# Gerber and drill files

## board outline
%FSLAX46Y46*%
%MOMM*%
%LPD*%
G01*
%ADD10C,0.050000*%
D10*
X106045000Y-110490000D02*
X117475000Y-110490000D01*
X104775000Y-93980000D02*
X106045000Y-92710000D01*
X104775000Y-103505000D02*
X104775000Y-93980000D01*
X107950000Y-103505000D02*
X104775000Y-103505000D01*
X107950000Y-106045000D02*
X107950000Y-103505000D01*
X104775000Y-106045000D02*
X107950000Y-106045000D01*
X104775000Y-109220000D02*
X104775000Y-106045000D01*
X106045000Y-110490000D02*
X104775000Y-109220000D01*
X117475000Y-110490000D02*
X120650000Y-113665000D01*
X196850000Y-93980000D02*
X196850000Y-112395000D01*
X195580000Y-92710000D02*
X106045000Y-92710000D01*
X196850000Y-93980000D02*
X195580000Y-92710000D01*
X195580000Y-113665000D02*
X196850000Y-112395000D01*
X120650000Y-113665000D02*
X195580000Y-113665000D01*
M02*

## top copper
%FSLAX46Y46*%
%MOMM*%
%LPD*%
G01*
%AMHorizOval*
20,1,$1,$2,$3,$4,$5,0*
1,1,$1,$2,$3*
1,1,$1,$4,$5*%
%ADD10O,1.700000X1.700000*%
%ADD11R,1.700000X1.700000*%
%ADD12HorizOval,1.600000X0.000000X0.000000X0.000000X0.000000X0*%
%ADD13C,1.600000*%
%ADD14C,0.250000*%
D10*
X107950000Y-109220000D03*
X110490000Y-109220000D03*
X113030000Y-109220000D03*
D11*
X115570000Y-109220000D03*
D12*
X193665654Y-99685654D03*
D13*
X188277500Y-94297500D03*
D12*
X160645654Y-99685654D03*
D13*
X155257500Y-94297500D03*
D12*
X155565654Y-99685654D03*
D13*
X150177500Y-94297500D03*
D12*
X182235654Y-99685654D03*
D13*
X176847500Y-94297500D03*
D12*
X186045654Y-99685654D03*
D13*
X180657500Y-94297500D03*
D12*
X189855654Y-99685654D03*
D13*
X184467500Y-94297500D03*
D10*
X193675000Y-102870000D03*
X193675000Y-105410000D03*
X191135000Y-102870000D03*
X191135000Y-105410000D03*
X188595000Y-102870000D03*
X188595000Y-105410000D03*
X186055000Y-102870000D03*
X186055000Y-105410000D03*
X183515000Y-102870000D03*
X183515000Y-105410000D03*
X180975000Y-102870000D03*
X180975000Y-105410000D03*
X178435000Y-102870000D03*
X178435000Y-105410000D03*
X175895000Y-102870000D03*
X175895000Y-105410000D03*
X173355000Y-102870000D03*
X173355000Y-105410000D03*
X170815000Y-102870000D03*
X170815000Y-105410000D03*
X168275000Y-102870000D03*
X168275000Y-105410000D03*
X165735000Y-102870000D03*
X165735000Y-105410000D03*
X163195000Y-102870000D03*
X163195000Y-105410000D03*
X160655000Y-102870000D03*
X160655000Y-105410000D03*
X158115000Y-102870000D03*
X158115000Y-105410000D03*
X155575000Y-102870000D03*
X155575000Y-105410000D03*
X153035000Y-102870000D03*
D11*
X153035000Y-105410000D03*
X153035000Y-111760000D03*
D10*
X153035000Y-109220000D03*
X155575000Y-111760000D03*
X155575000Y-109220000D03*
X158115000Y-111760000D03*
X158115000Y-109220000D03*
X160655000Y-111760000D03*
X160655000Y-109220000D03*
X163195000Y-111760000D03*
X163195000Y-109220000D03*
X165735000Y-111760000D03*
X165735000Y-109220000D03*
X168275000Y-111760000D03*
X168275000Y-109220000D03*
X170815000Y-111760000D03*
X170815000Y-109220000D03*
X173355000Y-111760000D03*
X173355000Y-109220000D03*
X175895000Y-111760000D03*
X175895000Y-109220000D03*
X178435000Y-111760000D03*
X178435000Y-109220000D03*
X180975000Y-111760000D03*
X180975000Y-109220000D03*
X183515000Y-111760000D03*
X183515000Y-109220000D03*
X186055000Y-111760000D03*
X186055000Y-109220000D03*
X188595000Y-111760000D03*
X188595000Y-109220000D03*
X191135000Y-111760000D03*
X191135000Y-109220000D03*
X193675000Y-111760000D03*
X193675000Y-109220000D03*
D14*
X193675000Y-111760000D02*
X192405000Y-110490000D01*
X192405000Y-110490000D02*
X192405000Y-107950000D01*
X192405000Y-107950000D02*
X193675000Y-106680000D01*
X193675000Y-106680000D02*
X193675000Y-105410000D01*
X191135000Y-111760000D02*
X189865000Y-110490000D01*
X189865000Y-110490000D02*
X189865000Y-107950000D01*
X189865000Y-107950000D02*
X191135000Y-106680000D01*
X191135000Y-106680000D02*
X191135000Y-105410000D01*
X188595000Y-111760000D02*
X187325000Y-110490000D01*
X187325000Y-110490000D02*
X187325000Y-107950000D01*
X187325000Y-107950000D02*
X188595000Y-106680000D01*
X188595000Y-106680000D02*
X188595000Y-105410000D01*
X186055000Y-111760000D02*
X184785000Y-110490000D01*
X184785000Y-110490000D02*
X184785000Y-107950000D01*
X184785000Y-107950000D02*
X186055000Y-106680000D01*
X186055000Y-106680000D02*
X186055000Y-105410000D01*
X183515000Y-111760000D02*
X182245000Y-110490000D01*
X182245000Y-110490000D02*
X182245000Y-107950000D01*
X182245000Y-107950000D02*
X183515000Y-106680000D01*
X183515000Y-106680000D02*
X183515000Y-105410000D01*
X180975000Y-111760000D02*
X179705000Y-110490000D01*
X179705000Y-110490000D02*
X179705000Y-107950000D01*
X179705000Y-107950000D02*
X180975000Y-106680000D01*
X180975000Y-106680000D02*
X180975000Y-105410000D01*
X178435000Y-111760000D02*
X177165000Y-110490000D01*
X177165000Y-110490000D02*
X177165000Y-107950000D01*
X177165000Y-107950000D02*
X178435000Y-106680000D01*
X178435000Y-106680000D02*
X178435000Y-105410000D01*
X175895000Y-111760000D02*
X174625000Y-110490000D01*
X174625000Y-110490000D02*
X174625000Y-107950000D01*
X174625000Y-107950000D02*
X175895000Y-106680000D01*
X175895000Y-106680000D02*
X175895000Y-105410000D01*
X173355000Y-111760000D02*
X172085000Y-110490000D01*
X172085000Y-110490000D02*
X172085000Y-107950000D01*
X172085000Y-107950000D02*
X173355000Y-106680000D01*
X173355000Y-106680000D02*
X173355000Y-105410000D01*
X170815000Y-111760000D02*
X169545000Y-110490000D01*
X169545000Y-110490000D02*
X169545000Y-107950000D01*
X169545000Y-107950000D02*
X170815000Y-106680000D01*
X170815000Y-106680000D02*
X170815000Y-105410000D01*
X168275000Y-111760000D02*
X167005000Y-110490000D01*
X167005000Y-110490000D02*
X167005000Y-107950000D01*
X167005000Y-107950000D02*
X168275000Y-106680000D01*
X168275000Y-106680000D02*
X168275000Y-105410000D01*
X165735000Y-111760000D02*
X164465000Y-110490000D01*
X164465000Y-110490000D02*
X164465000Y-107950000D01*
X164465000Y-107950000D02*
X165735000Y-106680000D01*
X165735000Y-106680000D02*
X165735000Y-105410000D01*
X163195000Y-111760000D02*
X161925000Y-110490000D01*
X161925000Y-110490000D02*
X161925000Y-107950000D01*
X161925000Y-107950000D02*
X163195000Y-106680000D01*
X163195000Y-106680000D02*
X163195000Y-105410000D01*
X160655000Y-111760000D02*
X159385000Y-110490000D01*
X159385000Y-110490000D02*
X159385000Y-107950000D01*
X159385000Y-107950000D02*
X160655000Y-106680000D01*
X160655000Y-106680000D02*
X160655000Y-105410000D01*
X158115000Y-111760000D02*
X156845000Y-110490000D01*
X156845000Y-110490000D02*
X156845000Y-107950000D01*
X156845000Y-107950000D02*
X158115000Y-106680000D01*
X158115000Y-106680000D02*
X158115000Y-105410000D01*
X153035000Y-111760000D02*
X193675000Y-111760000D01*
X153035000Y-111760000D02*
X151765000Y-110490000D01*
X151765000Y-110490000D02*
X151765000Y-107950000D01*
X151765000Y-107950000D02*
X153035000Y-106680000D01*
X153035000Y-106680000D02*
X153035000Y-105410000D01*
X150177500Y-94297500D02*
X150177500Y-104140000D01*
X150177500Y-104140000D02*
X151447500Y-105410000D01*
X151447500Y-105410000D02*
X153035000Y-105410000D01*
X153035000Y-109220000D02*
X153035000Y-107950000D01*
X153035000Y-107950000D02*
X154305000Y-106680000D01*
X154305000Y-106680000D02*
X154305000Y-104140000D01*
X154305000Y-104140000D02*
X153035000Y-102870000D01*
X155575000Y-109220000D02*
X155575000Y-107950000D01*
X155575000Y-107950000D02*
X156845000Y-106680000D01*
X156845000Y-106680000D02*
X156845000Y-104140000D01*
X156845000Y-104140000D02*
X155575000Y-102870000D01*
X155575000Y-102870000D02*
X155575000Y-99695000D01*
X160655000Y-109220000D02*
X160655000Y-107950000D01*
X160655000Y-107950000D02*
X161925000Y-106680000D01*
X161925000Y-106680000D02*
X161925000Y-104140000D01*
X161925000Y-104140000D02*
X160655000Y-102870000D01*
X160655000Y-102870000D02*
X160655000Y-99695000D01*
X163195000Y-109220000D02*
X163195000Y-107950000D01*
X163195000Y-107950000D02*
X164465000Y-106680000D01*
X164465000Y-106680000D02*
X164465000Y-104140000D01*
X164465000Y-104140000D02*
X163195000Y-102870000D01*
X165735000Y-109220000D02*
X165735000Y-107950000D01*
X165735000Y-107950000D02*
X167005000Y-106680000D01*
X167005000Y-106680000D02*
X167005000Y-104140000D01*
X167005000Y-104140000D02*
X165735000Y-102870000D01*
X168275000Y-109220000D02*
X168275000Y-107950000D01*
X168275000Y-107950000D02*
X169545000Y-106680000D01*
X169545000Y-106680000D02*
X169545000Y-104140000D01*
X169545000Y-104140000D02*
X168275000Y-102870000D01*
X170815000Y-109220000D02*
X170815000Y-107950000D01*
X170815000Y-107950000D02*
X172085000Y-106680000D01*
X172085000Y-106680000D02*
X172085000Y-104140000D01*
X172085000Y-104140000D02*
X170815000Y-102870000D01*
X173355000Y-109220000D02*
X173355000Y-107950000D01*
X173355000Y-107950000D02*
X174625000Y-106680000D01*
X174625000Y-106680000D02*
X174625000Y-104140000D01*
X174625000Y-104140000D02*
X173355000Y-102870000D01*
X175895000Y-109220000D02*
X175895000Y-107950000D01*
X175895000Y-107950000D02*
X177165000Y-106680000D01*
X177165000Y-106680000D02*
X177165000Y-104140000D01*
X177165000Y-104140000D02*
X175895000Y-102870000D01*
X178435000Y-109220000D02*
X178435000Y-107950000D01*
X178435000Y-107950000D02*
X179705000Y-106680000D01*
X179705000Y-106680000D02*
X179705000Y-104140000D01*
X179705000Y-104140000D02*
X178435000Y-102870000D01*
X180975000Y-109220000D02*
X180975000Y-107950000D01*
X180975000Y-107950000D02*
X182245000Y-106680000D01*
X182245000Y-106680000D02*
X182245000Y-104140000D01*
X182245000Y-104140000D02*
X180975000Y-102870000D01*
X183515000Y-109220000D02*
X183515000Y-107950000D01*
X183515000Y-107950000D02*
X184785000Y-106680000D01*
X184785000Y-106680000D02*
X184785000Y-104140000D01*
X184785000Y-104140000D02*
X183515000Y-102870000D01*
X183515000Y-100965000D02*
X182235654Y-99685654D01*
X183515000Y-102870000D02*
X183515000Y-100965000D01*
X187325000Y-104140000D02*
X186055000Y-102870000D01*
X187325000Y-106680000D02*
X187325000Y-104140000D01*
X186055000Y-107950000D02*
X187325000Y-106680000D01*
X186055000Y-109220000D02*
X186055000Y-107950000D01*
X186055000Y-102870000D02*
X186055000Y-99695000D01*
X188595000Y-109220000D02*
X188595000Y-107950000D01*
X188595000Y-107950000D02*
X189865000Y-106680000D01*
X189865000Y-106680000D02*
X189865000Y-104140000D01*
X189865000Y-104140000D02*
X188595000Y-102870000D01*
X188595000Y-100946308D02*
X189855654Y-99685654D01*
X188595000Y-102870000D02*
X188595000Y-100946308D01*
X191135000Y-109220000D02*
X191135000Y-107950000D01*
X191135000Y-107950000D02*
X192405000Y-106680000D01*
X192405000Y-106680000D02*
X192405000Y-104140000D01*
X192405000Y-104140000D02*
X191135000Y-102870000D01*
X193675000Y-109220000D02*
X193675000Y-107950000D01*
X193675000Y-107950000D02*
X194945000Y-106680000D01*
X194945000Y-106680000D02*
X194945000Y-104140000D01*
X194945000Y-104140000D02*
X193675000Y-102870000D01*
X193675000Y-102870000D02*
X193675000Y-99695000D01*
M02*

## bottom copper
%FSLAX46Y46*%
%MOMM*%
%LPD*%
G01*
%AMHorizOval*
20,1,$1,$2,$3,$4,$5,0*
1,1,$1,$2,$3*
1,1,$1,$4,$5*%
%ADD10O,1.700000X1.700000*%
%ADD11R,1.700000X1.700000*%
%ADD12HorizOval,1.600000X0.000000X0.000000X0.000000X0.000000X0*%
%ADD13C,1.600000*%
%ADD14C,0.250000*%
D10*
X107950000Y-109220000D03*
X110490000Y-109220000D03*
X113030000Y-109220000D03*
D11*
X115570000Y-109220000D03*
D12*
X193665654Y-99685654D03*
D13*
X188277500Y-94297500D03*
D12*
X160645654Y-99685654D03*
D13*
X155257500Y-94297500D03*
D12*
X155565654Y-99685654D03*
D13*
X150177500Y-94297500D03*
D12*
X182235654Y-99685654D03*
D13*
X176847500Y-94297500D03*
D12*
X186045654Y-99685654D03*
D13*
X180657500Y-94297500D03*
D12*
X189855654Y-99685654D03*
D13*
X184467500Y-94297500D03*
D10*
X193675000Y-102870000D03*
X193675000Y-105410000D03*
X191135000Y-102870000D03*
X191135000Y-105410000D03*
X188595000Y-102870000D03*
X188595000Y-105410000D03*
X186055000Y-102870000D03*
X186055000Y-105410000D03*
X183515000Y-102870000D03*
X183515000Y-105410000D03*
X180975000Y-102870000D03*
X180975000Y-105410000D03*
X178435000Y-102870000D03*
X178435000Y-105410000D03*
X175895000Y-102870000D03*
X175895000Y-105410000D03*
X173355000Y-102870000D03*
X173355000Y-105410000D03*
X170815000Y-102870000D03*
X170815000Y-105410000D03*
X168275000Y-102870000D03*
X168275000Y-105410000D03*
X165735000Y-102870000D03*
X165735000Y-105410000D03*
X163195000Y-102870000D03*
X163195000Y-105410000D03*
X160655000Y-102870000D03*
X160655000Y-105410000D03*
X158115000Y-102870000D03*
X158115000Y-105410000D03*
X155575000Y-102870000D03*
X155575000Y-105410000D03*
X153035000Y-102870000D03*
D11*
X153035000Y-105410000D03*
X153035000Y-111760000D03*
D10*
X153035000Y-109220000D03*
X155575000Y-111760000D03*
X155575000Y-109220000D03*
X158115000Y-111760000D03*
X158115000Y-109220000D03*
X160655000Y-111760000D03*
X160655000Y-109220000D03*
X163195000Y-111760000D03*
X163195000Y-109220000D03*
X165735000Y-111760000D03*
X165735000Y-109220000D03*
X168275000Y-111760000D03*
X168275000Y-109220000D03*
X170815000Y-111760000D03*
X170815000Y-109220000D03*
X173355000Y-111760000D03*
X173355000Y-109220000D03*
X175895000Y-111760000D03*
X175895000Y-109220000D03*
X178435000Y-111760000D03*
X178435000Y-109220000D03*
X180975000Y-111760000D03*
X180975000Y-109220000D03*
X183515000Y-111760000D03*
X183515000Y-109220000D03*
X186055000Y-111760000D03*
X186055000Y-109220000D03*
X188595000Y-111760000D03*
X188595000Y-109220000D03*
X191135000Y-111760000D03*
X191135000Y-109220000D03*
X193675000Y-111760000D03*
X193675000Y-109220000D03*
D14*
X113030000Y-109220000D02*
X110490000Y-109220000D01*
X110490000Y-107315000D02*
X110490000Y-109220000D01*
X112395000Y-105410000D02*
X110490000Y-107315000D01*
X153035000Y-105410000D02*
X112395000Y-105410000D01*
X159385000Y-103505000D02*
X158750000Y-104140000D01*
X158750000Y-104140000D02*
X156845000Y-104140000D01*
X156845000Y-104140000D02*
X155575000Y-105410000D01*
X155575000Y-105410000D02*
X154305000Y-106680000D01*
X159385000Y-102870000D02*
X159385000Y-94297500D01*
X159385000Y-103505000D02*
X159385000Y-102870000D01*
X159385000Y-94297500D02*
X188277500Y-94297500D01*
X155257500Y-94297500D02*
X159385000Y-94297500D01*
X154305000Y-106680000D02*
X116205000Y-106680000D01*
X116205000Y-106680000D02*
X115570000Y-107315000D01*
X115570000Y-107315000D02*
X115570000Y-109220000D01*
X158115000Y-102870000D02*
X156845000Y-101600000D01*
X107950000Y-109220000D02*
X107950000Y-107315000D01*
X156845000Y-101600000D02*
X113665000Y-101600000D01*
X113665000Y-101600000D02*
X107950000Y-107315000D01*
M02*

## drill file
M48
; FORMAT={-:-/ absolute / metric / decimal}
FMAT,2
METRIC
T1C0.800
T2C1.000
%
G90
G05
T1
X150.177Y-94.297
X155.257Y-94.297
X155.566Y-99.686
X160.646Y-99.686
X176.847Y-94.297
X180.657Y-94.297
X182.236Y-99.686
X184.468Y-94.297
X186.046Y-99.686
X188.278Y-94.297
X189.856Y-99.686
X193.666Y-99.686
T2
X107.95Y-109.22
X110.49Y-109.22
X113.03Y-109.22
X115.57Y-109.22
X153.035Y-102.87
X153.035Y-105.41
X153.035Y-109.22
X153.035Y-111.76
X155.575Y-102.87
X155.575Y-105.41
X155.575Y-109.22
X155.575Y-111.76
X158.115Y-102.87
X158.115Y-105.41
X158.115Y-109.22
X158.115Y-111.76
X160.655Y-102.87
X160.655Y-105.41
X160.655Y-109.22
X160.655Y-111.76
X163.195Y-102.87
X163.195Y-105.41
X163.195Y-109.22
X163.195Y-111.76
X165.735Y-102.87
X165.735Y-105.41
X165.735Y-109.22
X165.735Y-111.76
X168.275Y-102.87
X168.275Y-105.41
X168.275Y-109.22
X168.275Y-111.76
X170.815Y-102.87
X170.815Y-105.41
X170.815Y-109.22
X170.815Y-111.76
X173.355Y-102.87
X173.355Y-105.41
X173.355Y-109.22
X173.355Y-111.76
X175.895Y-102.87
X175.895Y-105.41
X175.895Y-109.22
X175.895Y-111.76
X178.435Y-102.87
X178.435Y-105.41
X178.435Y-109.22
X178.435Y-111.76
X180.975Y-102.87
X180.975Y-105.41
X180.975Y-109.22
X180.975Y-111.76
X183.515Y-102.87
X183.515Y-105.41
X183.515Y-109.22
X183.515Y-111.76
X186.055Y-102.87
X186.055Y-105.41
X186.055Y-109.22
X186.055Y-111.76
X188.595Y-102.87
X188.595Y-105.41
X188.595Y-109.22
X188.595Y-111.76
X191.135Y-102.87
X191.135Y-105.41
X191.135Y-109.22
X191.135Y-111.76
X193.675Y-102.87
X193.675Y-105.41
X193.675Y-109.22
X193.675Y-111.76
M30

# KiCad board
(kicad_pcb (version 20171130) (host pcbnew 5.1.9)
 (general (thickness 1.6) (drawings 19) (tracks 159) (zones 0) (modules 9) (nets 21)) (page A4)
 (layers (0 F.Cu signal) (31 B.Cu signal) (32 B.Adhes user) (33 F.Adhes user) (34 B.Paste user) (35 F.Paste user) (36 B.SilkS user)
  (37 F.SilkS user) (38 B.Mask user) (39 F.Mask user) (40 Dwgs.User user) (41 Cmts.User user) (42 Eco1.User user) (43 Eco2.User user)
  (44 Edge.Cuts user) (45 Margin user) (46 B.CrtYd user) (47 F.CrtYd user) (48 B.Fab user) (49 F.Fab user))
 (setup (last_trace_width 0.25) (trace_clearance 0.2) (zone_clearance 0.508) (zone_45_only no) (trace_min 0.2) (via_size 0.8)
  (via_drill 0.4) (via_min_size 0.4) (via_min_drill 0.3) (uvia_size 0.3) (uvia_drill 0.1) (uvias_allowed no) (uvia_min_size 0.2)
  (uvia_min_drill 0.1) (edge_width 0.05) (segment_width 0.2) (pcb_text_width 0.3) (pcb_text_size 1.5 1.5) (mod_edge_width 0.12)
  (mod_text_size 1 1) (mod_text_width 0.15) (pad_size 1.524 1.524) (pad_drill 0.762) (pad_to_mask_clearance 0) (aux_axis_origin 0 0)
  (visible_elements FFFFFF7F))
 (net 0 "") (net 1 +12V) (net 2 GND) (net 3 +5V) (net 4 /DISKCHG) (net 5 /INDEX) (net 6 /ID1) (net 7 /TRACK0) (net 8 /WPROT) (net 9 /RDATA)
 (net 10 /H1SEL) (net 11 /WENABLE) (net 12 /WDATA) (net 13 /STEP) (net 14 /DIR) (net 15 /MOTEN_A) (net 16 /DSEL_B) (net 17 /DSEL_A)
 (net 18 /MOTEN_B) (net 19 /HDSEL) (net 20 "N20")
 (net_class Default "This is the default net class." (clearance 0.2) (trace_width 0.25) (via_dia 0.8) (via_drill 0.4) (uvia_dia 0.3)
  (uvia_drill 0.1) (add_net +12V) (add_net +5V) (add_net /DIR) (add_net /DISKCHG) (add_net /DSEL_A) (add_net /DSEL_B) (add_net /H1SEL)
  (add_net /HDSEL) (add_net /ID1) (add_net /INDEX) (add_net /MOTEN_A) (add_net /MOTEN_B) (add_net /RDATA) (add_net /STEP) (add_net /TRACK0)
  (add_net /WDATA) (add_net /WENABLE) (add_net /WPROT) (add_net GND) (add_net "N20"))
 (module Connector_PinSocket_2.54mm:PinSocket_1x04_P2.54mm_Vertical (layer B.Cu) (at 115.57 109.22 90)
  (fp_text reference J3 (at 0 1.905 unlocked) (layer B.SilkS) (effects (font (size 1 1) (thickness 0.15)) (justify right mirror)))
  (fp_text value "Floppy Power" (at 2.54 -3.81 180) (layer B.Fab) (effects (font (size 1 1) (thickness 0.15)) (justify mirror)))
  (pad 4 thru_hole oval (at 0 -7.62 90) (size 1.7 1.7) (drill 1) (layers *.Cu *.Mask) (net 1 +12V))
  (pad 3 thru_hole oval (at 0 -5.08 90) (size 1.7 1.7) (drill 1) (layers *.Cu *.Mask) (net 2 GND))
  (pad 2 thru_hole oval (at 0 -2.54 90) (size 1.7 1.7) (drill 1) (layers *.Cu *.Mask) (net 2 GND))
  (pad 1 thru_hole rect (at 0 0 90) (size 1.7 1.7) (drill 1) (layers *.Cu *.Mask) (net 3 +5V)))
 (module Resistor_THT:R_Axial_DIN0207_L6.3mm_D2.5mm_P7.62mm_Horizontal (layer F.Cu) (at 188.2775 94.2975 315)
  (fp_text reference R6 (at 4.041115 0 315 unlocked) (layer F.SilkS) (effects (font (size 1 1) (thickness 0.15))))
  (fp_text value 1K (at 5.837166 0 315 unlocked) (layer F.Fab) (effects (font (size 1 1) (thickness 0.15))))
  (pad 2 thru_hole oval (at 7.62 0 315) (size 1.6 1.6) (drill 0.8) (layers *.Cu *.Mask) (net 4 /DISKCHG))
  (pad 1 thru_hole circle (at 0 0 315) (size 1.6 1.6) (drill 0.8) (layers *.Cu *.Mask) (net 3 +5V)))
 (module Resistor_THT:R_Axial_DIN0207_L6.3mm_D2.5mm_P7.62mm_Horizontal (layer F.Cu) (at 155.2575 94.2975 315)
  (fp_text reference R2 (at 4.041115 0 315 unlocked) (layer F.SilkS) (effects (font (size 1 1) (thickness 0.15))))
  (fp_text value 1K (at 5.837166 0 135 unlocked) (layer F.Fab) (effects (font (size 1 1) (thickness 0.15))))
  (pad 2 thru_hole oval (at 7.62 0 315) (size 1.6 1.6) (drill 0.8) (layers *.Cu *.Mask) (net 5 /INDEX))
  (pad 1 thru_hole circle (at 0 0 315) (size 1.6 1.6) (drill 0.8) (layers *.Cu *.Mask) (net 3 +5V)))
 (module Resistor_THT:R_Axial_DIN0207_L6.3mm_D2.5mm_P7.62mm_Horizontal (layer F.Cu) (at 150.1775 94.2975 315)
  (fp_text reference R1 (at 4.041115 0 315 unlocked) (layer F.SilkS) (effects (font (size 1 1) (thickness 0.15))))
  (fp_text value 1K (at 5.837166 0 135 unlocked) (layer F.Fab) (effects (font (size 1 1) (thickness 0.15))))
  (pad 2 thru_hole oval (at 7.62 0 315) (size 1.6 1.6) (drill 0.8) (layers *.Cu *.Mask) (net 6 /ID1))
  (pad 1 thru_hole circle (at 0 0 315) (size 1.6 1.6) (drill 0.8) (layers *.Cu *.Mask) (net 2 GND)))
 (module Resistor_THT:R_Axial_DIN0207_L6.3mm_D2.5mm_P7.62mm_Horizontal (layer F.Cu) (at 176.8475 94.2975 315)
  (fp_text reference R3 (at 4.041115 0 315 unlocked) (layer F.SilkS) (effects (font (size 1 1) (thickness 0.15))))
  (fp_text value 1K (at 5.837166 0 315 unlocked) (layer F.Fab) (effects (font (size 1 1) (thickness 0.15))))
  (pad 2 thru_hole oval (at 7.62 0 315) (size 1.6 1.6) (drill 0.8) (layers *.Cu *.Mask) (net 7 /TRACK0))
  (pad 1 thru_hole circle (at 0 0 315) (size 1.6 1.6) (drill 0.8) (layers *.Cu *.Mask) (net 3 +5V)))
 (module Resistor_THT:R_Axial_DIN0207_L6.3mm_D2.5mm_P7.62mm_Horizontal (layer F.Cu) (at 180.6575 94.2975 315)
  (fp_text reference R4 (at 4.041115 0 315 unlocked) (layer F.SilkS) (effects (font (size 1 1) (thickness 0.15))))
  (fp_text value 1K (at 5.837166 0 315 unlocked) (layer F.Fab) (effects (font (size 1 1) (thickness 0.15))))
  (pad 2 thru_hole oval (at 7.62 0 315) (size 1.6 1.6) (drill 0.8) (layers *.Cu *.Mask) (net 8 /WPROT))
  (pad 1 thru_hole circle (at 0 0 315) (size 1.6 1.6) (drill 0.8) (layers *.Cu *.Mask) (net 3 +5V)))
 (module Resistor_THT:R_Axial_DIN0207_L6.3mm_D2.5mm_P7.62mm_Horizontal (layer F.Cu) (at 184.4675 94.2975 315)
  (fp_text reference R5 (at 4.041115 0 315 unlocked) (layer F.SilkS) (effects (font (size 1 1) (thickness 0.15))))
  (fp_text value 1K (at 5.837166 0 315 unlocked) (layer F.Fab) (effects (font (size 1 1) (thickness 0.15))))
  (pad 2 thru_hole oval (at 7.62 0 315) (size 1.6 1.6) (drill 0.8) (layers *.Cu *.Mask) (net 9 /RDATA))
  (pad 1 thru_hole circle (at 0 0 315) (size 1.6 1.6) (drill 0.8) (layers *.Cu *.Mask) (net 3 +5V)))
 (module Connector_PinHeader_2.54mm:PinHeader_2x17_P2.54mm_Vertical (layer F.Cu) (at 153.035 105.41 90)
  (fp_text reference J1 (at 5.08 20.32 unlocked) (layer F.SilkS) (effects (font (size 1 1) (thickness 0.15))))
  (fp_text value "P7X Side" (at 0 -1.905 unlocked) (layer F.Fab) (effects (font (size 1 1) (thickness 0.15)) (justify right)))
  (pad 34 thru_hole oval (at 2.54 40.64 90) (size 1.7 1.7) (drill 1) (layers *.Cu *.Mask) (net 4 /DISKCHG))
  (pad 33 thru_hole oval (at 0 40.64 90) (size 1.7 1.7) (drill 1) (layers *.Cu *.Mask) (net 2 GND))
  (pad 32 thru_hole oval (at 2.54 38.1 90) (size 1.7 1.7) (drill 1) (layers *.Cu *.Mask) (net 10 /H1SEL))
  (pad 31 thru_hole oval (at 0 38.1 90) (size 1.7 1.7) (drill 1) (layers *.Cu *.Mask) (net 2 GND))
  (pad 30 thru_hole oval (at 2.54 35.56 90) (size 1.7 1.7) (drill 1) (layers *.Cu *.Mask) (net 9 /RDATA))
  (pad 29 thru_hole oval (at 0 35.56 90) (size 1.7 1.7) (drill 1) (layers *.Cu *.Mask) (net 2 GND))
  (pad 28 thru_hole oval (at 2.54 33.02 90) (size 1.7 1.7) (drill 1) (layers *.Cu *.Mask) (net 8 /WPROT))
  (pad 27 thru_hole oval (at 0 33.02 90) (size 1.7 1.7) (drill 1) (layers *.Cu *.Mask) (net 2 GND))
  (pad 26 thru_hole oval (at 2.54 30.48 90) (size 1.7 1.7) (drill 1) (layers *.Cu *.Mask) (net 7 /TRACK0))
  (pad 25 thru_hole oval (at 0 30.48 90) (size 1.7 1.7) (drill 1) (layers *.Cu *.Mask) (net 2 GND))
  (pad 24 thru_hole oval (at 2.54 27.94 90) (size 1.7 1.7) (drill 1) (layers *.Cu *.Mask) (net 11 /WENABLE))
  (pad 23 thru_hole oval (at 0 27.94 90) (size 1.7 1.7) (drill 1) (layers *.Cu *.Mask) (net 2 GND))
  (pad 22 thru_hole oval (at 2.54 25.4 90) (size 1.7 1.7) (drill 1) (layers *.Cu *.Mask) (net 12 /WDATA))
  (pad 21 thru_hole oval (at 0 25.4 90) (size 1.7 1.7) (drill 1) (layers *.Cu *.Mask) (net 2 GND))
  (pad 20 thru_hole oval (at 2.54 22.86 90) (size 1.7 1.7) (drill 1) (layers *.Cu *.Mask) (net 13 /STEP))
  (pad 19 thru_hole oval (at 0 22.86 90) (size 1.7 1.7) (drill 1) (layers *.Cu *.Mask) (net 2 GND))
  (pad 18 thru_hole oval (at 2.54 20.32 90) (size 1.7 1.7) (drill 1) (layers *.Cu *.Mask) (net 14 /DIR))
  (pad 17 thru_hole oval (at 0 20.32 90) (size 1.7 1.7) (drill 1) (layers *.Cu *.Mask) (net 2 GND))
  (pad 16 thru_hole oval (at 2.54 17.78 90) (size 1.7 1.7) (drill 1) (layers *.Cu *.Mask) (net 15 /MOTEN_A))
  (pad 15 thru_hole oval (at 0 17.78 90) (size 1.7 1.7) (drill 1) (layers *.Cu *.Mask) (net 2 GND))
  (pad 14 thru_hole oval (at 2.54 15.24 90) (size 1.7 1.7) (drill 1) (layers *.Cu *.Mask) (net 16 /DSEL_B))
  (pad 13 thru_hole oval (at 0 15.24 90) (size 1.7 1.7) (drill 1) (layers *.Cu *.Mask) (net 2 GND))
  (pad 12 thru_hole oval (at 2.54 12.7 90) (size 1.7 1.7) (drill 1) (layers *.Cu *.Mask) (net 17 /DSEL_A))
  (pad 11 thru_hole oval (at 0 12.7 90) (size 1.7 1.7) (drill 1) (layers *.Cu *.Mask) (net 2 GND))
  (pad 10 thru_hole oval (at 2.54 10.16 90) (size 1.7 1.7) (drill 1) (layers *.Cu *.Mask) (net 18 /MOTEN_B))
  (pad 9 thru_hole oval (at 0 10.16 90) (size 1.7 1.7) (drill 1) (layers *.Cu *.Mask) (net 2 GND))
  (pad 8 thru_hole oval (at 2.54 7.62 90) (size 1.7 1.7) (drill 1) (layers *.Cu *.Mask) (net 5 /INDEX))
  (pad 7 thru_hole oval (at 0 7.62 90) (size 1.7 1.7) (drill 1) (layers *.Cu *.Mask) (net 2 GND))
  (pad 6 thru_hole oval (at 2.54 5.08 90) (size 1.7 1.7) (drill 1) (layers *.Cu *.Mask) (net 1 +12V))
  (pad 5 thru_hole oval (at 0 5.08 90) (size 1.7 1.7) (drill 1) (layers *.Cu *.Mask) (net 2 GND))
  (pad 4 thru_hole oval (at 2.54 2.54 90) (size 1.7 1.7) (drill 1) (layers *.Cu *.Mask) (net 6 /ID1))
  (pad 3 thru_hole oval (at 0 2.54 90) (size 1.7 1.7) (drill 1) (layers *.Cu *.Mask) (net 3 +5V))
  (pad 2 thru_hole oval (at 2.54 0 90) (size 1.7 1.7) (drill 1) (layers *.Cu *.Mask) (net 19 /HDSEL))
  (pad 1 thru_hole rect (at 0 0 90) (size 1.7 1.7) (drill 1) (layers *.Cu *.Mask) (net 2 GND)))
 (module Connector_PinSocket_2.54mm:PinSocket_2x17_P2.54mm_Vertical (layer B.Cu) (at 153.035 111.76 270)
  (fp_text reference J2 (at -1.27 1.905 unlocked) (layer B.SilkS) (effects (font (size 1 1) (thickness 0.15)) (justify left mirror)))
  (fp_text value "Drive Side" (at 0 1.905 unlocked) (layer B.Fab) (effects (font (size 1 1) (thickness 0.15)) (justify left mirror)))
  (pad 1 thru_hole rect (at 0 0 270) (size 1.7 1.7) (drill 1) (layers *.Cu *.Mask) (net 2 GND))
  (pad 2 thru_hole oval (at -2.54 0 270) (size 1.7 1.7) (drill 1) (layers *.Cu *.Mask) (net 19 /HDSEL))
  (pad 3 thru_hole oval (at 0 -2.54 270) (size 1.7 1.7) (drill 1) (layers *.Cu *.Mask) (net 2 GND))
  (pad 4 thru_hole oval (at -2.54 -2.54 270) (size 1.7 1.7) (drill 1) (layers *.Cu *.Mask) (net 6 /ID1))
  (pad 5 thru_hole oval (at 0 -5.08 270) (size 1.7 1.7) (drill 1) (layers *.Cu *.Mask) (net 2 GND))
  (pad 6 thru_hole oval (at -2.54 -5.08 270) (size 1.7 1.7) (drill 1) (layers *.Cu *.Mask) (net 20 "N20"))
  (pad 7 thru_hole oval (at 0 -7.62 270) (size 1.7 1.7) (drill 1) (layers *.Cu *.Mask) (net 2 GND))
  (pad 8 thru_hole oval (at -2.54 -7.62 270) (size 1.7 1.7) (drill 1) (layers *.Cu *.Mask) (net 5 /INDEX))
  (pad 9 thru_hole oval (at 0 -10.16 270) (size 1.7 1.7) (drill 1) (layers *.Cu *.Mask) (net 2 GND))
  (pad 10 thru_hole oval (at -2.54 -10.16 270) (size 1.7 1.7) (drill 1) (layers *.Cu *.Mask) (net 18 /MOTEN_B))
  (pad 11 thru_hole oval (at 0 -12.7 270) (size 1.7 1.7) (drill 1) (layers *.Cu *.Mask) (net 2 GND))
  (pad 12 thru_hole oval (at -2.54 -12.7 270) (size 1.7 1.7) (drill 1) (layers *.Cu *.Mask) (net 17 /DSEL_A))
  (pad 13 thru_hole oval (at 0 -15.24 270) (size 1.7 1.7) (drill 1) (layers *.Cu *.Mask) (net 2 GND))
  (pad 14 thru_hole oval (at -2.54 -15.24 270) (size 1.7 1.7) (drill 1) (layers *.Cu *.Mask) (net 16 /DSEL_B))
  (pad 15 thru_hole oval (at 0 -17.78 270) (size 1.7 1.7) (drill 1) (layers *.Cu *.Mask) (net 2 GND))
  (pad 16 thru_hole oval (at -2.54 -17.78 270) (size 1.7 1.7) (drill 1) (layers *.Cu *.Mask) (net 15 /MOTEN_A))
  (pad 17 thru_hole oval (at 0 -20.32 270) (size 1.7 1.7) (drill 1) (layers *.Cu *.Mask) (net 2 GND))
  (pad 18 thru_hole oval (at -2.54 -20.32 270) (size 1.7 1.7) (drill 1) (layers *.Cu *.Mask) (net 14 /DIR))
  (pad 19 thru_hole oval (at 0 -22.86 270) (size 1.7 1.7) (drill 1) (layers *.Cu *.Mask) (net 2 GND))
  (pad 20 thru_hole oval (at -2.54 -22.86 270) (size 1.7 1.7) (drill 1) (layers *.Cu *.Mask) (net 13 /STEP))
  (pad 21 thru_hole oval (at 0 -25.4 270) (size 1.7 1.7) (drill 1) (layers *.Cu *.Mask) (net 2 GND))
  (pad 22 thru_hole oval (at -2.54 -25.4 270) (size 1.7 1.7) (drill 1) (layers *.Cu *.Mask) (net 12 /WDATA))
  (pad 23 thru_hole oval (at 0 -27.94 270) (size 1.7 1.7) (drill 1) (layers *.Cu *.Mask) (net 2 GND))
  (pad 24 thru_hole oval (at -2.54 -27.94 270) (size 1.7 1.7) (drill 1) (layers *.Cu *.Mask) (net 11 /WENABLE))
  (pad 25 thru_hole oval (at 0 -30.48 270) (size 1.7 1.7) (drill 1) (layers *.Cu *.Mask) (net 2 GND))
  (pad 26 thru_hole oval (at -2.54 -30.48 270) (size 1.7 1.7) (drill 1) (layers *.Cu *.Mask) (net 7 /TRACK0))
  (pad 27 thru_hole oval (at 0 -33.02 270) (size 1.7 1.7) (drill 1) (layers *.Cu *.Mask) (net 2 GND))
  (pad 28 thru_hole oval (at -2.54 -33.02 270) (size 1.7 1.7) (drill 1) (layers *.Cu *.Mask) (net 8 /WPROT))
  (pad 29 thru_hole oval (at 0 -35.56 270) (size 1.7 1.7) (drill 1) (layers *.Cu *.Mask) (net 2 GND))
  (pad 30 thru_hole oval (at -2.54 -35.56 270) (size 1.7 1.7) (drill 1) (layers *.Cu *.Mask) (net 9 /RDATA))
  (pad 31 thru_hole oval (at 0 -38.1 270) (size 1.7 1.7) (drill 1) (layers *.Cu *.Mask) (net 2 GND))
  (pad 32 thru_hole oval (at -2.54 -38.1 270) (size 1.7 1.7) (drill 1) (layers *.Cu *.Mask) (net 10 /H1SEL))
  (pad 33 thru_hole oval (at 0 -40.64 270) (size 1.7 1.7) (drill 1) (layers *.Cu *.Mask) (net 2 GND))
  (pad 34 thru_hole oval (at -2.54 -40.64 270) (size 1.7 1.7) (drill 1) (layers *.Cu *.Mask) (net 4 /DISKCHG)))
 (gr_line (start 106.045 110.49) (end 117.475 110.49) (layer Edge.Cuts) (width 0.05))
 (gr_line (start 104.775 93.98) (end 106.045 92.71) (layer Edge.Cuts) (width 0.05))
 (gr_line (start 104.775 103.505) (end 104.775 93.98) (layer Edge.Cuts) (width 0.05))
 (gr_line (start 107.95 103.505) (end 104.775 103.505) (layer Edge.Cuts) (width 0.05))
 (gr_line (start 107.95 106.045) (end 107.95 103.505) (layer Edge.Cuts) (width 0.05))
 (gr_line (start 104.775 106.045) (end 107.95 106.045) (layer Edge.Cuts) (width 0.05))
 (gr_line (start 104.775 109.22) (end 104.775 106.045) (layer Edge.Cuts) (width 0.05))
 (gr_line (start 106.045 110.49) (end 104.775 109.22) (layer Edge.Cuts) (width 0.05))
 (gr_line (start 117.475 110.49) (end 120.65 113.665) (layer Edge.Cuts) (width 0.05))
 (gr_line (start 196.85 93.98) (end 196.85 112.395) (layer Edge.Cuts) (width 0.05))
 (gr_line (start 195.58 92.71) (end 106.045 92.71) (layer Edge.Cuts) (width 0.05))
 (gr_line (start 196.85 93.98) (end 195.58 92.71) (layer Edge.Cuts) (width 0.05))
 (gr_line (start 195.58 113.665) (end 196.85 112.395) (layer Edge.Cuts) (width 0.05))
 (gr_line (start 120.65 113.665) (end 195.58 113.665) (layer Edge.Cuts) (width 0.05))
 (segment (start 193.675 111.76) (end 192.405 110.49) (width 0.25) (layer F.Cu) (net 2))
 (segment (start 192.405 110.49) (end 192.405 107.95) (width 0.25) (layer F.Cu) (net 2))
 (segment (start 192.405 107.95) (end 193.675 106.68) (width 0.25) (layer F.Cu) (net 2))
 (segment (start 193.675 106.68) (end 193.675 105.41) (width 0.25) (layer F.Cu) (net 2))
 (segment (start 191.135 111.76) (end 189.865 110.49) (width 0.25) (layer F.Cu) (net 2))
 (segment (start 189.865 110.49) (end 189.865 107.95) (width 0.25) (layer F.Cu) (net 2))
 (segment (start 189.865 107.95) (end 191.135 106.68) (width 0.25) (layer F.Cu) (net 2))
 (segment (start 191.135 106.68) (end 191.135 105.41) (width 0.25) (layer F.Cu) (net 2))
 (segment (start 188.595 111.76) (end 187.325 110.49) (width 0.25) (layer F.Cu) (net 2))
 (segment (start 187.325 110.49) (end 187.325 107.95) (width 0.25) (layer F.Cu) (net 2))
 (segment (start 187.325 107.95) (end 188.595 106.68) (width 0.25) (layer F.Cu) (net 2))
 (segment (start 188.595 106.68) (end 188.595 105.41) (width 0.25) (layer F.Cu) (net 2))
 (segment (start 186.055 111.76) (end 184.785 110.49) (width 0.25) (layer F.Cu) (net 2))
 (segment (start 184.785 110.49) (end 184.785 107.95) (width 0.25) (layer F.Cu) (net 2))
 (segment (start 184.785 107.95) (end 186.055 106.68) (width 0.25) (layer F.Cu) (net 2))
 (segment (start 186.055 106.68) (end 186.055 105.41) (width 0.25) (layer F.Cu) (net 2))
 (segment (start 183.515 111.76) (end 182.245 110.49) (width 0.25) (layer F.Cu) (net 2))
 (segment (start 182.245 110.49) (end 182.245 107.95) (width 0.25) (layer F.Cu) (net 2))
 (segment (start 182.245 107.95) (end 183.515 106.68) (width 0.25) (layer F.Cu) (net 2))
 (segment (start 183.515 106.68) (end 183.515 105.41) (width 0.25) (layer F.Cu) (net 2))
 (segment (start 180.975 111.76) (end 179.705 110.49) (width 0.25) (layer F.Cu) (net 2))
 (segment (start 179.705 110.49) (end 179.705 107.95) (width 0.25) (layer F.Cu) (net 2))
 (segment (start 179.705 107.95) (end 180.975 106.68) (width 0.25) (layer F.Cu) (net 2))
 (segment (start 180.975 106.68) (end 180.975 105.41) (width 0.25) (layer F.Cu) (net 2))
 (segment (start 178.435 111.76) (end 177.165 110.49) (width 0.25) (layer F.Cu) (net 2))
 (segment (start 177.165 110.49) (end 177.165 107.95) (width 0.25) (layer F.Cu) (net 2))
 (segment (start 177.165 107.95) (end 178.435 106.68) (width 0.25) (layer F.Cu) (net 2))
 (segment (start 178.435 106.68) (end 178.435 105.41) (width 0.25) (layer F.Cu) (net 2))
 (segment (start 175.895 111.76) (end 174.625 110.49) (width 0.25) (layer F.Cu) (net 2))
 (segment (start 174.625 110.49) (end 174.625 107.95) (width 0.25) (layer F.Cu) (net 2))
 (segment (start 174.625 107.95) (end 175.895 106.68) (width 0.25) (layer F.Cu) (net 2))
 (segment (start 175.895 106.68) (end 175.895 105.41) (width 0.25) (layer F.Cu) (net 2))
 (segment (start 173.355 111.76) (end 172.085 110.49) (width 0.25) (layer F.Cu) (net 2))
 (segment (start 172.085 110.49) (end 172.085 107.95) (width 0.25) (layer F.Cu) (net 2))
 (segment (start 172.085 107.95) (end 173.355 106.68) (width 0.25) (layer F.Cu) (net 2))
 (segment (start 173.355 106.68) (end 173.355 105.41) (width 0.25) (layer F.Cu) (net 2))
 (segment (start 170.815 111.76) (end 169.545 110.49) (width 0.25) (layer F.Cu) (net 2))
 (segment (start 169.545 110.49) (end 169.545 107.95) (width 0.25) (layer F.Cu) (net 2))
 (segment (start 169.545 107.95) (end 170.815 106.68) (width 0.25) (layer F.Cu) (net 2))
 (segment (start 170.815 106.68) (end 170.815 105.41) (width 0.25) (layer F.Cu) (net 2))
 (segment (start 168.275 111.76) (end 167.005 110.49) (width 0.25) (layer F.Cu) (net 2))
 (segment (start 167.005 110.49) (end 167.005 107.95) (width 0.25) (layer F.Cu) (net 2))
 (segment (start 167.005 107.95) (end 168.275 106.68) (width 0.25) (layer F.Cu) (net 2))
 (segment (start 168.275 106.68) (end 168.275 105.41) (width 0.25) (layer F.Cu) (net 2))
 (segment (start 165.735 111.76) (end 164.465 110.49) (width 0.25) (layer F.Cu) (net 2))
 (segment (start 164.465 110.49) (end 164.465 107.95) (width 0.25) (layer F.Cu) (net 2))
 (segment (start 164.465 107.95) (end 165.735 106.68) (width 0.25) (layer F.Cu) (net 2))
 (segment (start 165.735 106.68) (end 165.735 105.41) (width 0.25) (layer F.Cu) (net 2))
 (segment (start 163.195 111.76) (end 161.925 110.49) (width 0.25) (layer F.Cu) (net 2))
 (segment (start 161.925 110.49) (end 161.925 107.95) (width 0.25) (layer F.Cu) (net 2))
 (segment (start 161.925 107.95) (end 163.195 106.68) (width 0.25) (layer F.Cu) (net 2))
 (segment (start 163.195 106.68) (end 163.195 105.41) (width 0.25) (layer F.Cu) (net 2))
 (segment (start 160.655 111.76) (end 159.385 110.49) (width 0.25) (layer F.Cu) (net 2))
 (segment (start 159.385 110.49) (end 159.385 107.95) (width 0.25) (layer F.Cu) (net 2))
 (segment (start 159.385 107.95) (end 160.655 106.68) (width 0.25) (layer F.Cu) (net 2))
 (segment (start 160.655 106.68) (end 160.655 105.41) (width 0.25) (layer F.Cu) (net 2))
 (segment (start 158.115 111.76) (end 156.845 110.49) (width 0.25) (layer F.Cu) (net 2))
 (segment (start 156.845 110.49) (end 156.845 107.95) (width 0.25) (layer F.Cu) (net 2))
 (segment (start 156.845 107.95) (end 158.115 106.68) (width 0.25) (layer F.Cu) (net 2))
 (segment (start 158.115 106.68) (end 158.115 105.41) (width 0.25) (layer F.Cu) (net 2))
 (segment (start 153.035 111.76) (end 193.675 111.76) (width 0.25) (layer F.Cu) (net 2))
 (segment (start 153.035 111.76) (end 151.765 110.49) (width 0.25) (layer F.Cu) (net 2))
 (segment (start 151.765 110.49) (end 151.765 107.95) (width 0.25) (layer F.Cu) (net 2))
 (segment (start 151.765 107.95) (end 153.035 106.68) (width 0.25) (layer F.Cu) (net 2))
 (segment (start 153.035 106.68) (end 153.035 105.41) (width 0.25) (layer F.Cu) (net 2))
 (segment (start 113.03 109.22) (end 110.49 109.22) (width 0.25) (layer B.Cu) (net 2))
 (segment (start 110.49 107.315) (end 110.49 109.22) (width 0.25) (layer B.Cu) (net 2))
 (segment (start 112.395 105.41) (end 110.49 107.315) (width 0.25) (layer B.Cu) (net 2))
 (segment (start 153.035 105.41) (end 112.395 105.41) (width 0.25) (layer B.Cu) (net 2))
 (segment (start 150.1775 94.2975) (end 150.1775 104.14) (width 0.25) (layer F.Cu) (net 2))
 (segment (start 150.1775 104.14) (end 151.4475 105.41) (width 0.25) (layer F.Cu) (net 2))
 (segment (start 151.4475 105.41) (end 153.035 105.41) (width 0.25) (layer F.Cu) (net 2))
 (segment (start 153.035 109.22) (end 153.035 107.95) (width 0.25) (layer F.Cu) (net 19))
 (segment (start 153.035 107.95) (end 154.305 106.68) (width 0.25) (layer F.Cu) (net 19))
 (segment (start 154.305 106.68) (end 154.305 104.14) (width 0.25) (layer F.Cu) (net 19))
 (segment (start 154.305 104.14) (end 153.035 102.87) (width 0.25) (layer F.Cu) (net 19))
 (segment (start 159.385 103.505) (end 158.75 104.14) (width 0.25) (layer B.Cu) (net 3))
 (segment (start 158.75 104.14) (end 156.845 104.14) (width 0.25) (layer B.Cu) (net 3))
 (segment (start 156.845 104.14) (end 155.575 105.41) (width 0.25) (layer B.Cu) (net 3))
 (segment (start 155.575 105.41) (end 154.305 106.68) (width 0.25) (layer B.Cu) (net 3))
 (segment (start 159.385 102.87) (end 159.385 94.2975) (width 0.25) (layer B.Cu) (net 3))
 (segment (start 159.385 103.505) (end 159.385 102.87) (width 0.25) (layer B.Cu) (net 3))
 (segment (start 159.385 94.2975) (end 188.2775 94.2975) (width 0.25) (layer B.Cu) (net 3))
 (segment (start 155.2575 94.2975) (end 159.385 94.2975) (width 0.25) (layer B.Cu) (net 3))
 (segment (start 154.305 106.68) (end 116.205 106.68) (width 0.25) (layer B.Cu) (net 3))
 (segment (start 116.205 106.68) (end 115.57 107.315) (width 0.25) (layer B.Cu) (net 3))
 (segment (start 115.57 107.315) (end 115.57 109.22) (width 0.25) (layer B.Cu) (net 3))
 (segment (start 155.575 109.22) (end 155.575 107.95) (width 0.25) (layer F.Cu) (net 6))
 (segment (start 155.575 107.95) (end 156.845 106.68) (width 0.25) (layer F.Cu) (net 6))
 (segment (start 156.845 106.68) (end 156.845 104.14) (width 0.25) (layer F.Cu) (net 6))
 (segment (start 156.845 104.14) (end 155.575 102.87) (width 0.25) (layer F.Cu) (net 6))
 (segment (start 155.575 102.87) (end 155.575 99.695) (width 0.25) (layer F.Cu) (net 6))
 (segment (start 158.115 102.87) (end 156.845 101.6) (width 0.25) (layer B.Cu) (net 1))
 (segment (start 107.95 109.22) (end 107.95 107.315) (width 0.25) (layer B.Cu) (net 1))
 (segment (start 156.845 101.6) (end 113.665 101.6) (width 0.25) (layer B.Cu) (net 1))
 (segment (start 113.665 101.6) (end 107.95 107.315) (width 0.25) (layer B.Cu) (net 1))
 (segment (start 160.655 109.22) (end 160.655 107.95) (width 0.25) (layer F.Cu) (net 5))
 (segment (start 160.655 107.95) (end 161.925 106.68) (width 0.25) (layer F.Cu) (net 5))
 (segment (start 161.925 106.68) (end 161.925 104.14) (width 0.25) (layer F.Cu) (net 5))
 (segment (start 161.925 104.14) (end 160.655 102.87) (width 0.25) (layer F.Cu) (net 5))
 (segment (start 160.655 102.87) (end 160.655 99.695) (width 0.25) (layer F.Cu) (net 5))
 (segment (start 163.195 109.22) (end 163.195 107.95) (width 0.25) (layer F.Cu) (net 18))
 (segment (start 163.195 107.95) (end 164.465 106.68) (width 0.25) (layer F.Cu) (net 18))
 (segment (start 164.465 106.68) (end 164.465 104.14) (width 0.25) (layer F.Cu) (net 18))
 (segment (start 164.465 104.14) (end 163.195 102.87) (width 0.25) (layer F.Cu) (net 18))
 (segment (start 165.735 109.22) (end 165.735 107.95) (width 0.25) (layer F.Cu) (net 17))
 (segment (start 165.735 107.95) (end 167.005 106.68) (width 0.25) (layer F.Cu) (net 17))
 (segment (start 167.005 106.68) (end 167.005 104.14) (width 0.25) (layer F.Cu) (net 17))
 (segment (start 167.005 104.14) (end 165.735 102.87) (width 0.25) (layer F.Cu) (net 17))
 (segment (start 168.275 109.22) (end 168.275 107.95) (width 0.25) (layer F.Cu) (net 16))
 (segment (start 168.275 107.95) (end 169.545 106.68) (width 0.25) (layer F.Cu) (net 16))
 (segment (start 169.545 106.68) (end 169.545 104.14) (width 0.25) (layer F.Cu) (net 16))
 (segment (start 169.545 104.14) (end 168.275 102.87) (width 0.25) (layer F.Cu) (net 16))
 (segment (start 170.815 109.22) (end 170.815 107.95) (width 0.25) (layer F.Cu) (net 15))
 (segment (start 170.815 107.95) (end 172.085 106.68) (width 0.25) (layer F.Cu) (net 15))
 (segment (start 172.085 106.68) (end 172.085 104.14) (width 0.25) (layer F.Cu) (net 15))
 (segment (start 172.085 104.14) (end 170.815 102.87) (width 0.25) (layer F.Cu) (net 15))
 (segment (start 173.355 109.22) (end 173.355 107.95) (width 0.25) (layer F.Cu) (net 14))
 (segment (start 173.355 107.95) (end 174.625 106.68) (width 0.25) (layer F.Cu) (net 14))
 (segment (start 174.625 106.68) (end 174.625 104.14) (width 0.25) (layer F.Cu) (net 14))
 (segment (start 174.625 104.14) (end 173.355 102.87) (width 0.25) (layer F.Cu) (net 14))
 (segment (start 175.895 109.22) (end 175.895 107.95) (width 0.25) (layer F.Cu) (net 13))
 (segment (start 175.895 107.95) (end 177.165 106.68) (width 0.25) (layer F.Cu) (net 13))
 (segment (start 177.165 106.68) (end 177.165 104.14) (width 0.25) (layer F.Cu) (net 13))
 (segment (start 177.165 104.14) (end 175.895 102.87) (width 0.25) (layer F.Cu) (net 13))
 (segment (start 178.435 109.22) (end 178.435 107.95) (width 0.25) (layer F.Cu) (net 12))
 (segment (start 178.435 107.95) (end 179.705 106.68) (width 0.25) (layer F.Cu) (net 12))
 (segment (start 179.705 106.68) (end 179.705 104.14) (width 0.25) (layer F.Cu) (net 12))
 (segment (start 179.705 104.14) (end 178.435 102.87) (width 0.25) (layer F.Cu) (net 12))
 (segment (start 180.975 109.22) (end 180.975 107.95) (width 0.25) (layer F.Cu) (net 11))
 (segment (start 180.975 107.95) (end 182.245 106.68) (width 0.25) (layer F.Cu) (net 11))
 (segment (start 182.245 106.68) (end 182.245 104.14) (width 0.25) (layer F.Cu) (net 11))
 (segment (start 182.245 104.14) (end 180.975 102.87) (width 0.25) (layer F.Cu) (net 11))
 (segment (start 183.515 109.22) (end 183.515 107.95) (width 0.25) (layer F.Cu) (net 7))
 (segment (start 183.515 107.95) (end 184.785 106.68) (width 0.25) (layer F.Cu) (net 7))
 (segment (start 184.785 106.68) (end 184.785 104.14) (width 0.25) (layer F.Cu) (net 7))
 (segment (start 184.785 104.14) (end 183.515 102.87) (width 0.25) (layer F.Cu) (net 7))
 (segment (start 183.515 100.965) (end 182.235654 99.685654) (width 0.25) (layer F.Cu) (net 7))
 (segment (start 183.515 102.87) (end 183.515 100.965) (width 0.25) (layer F.Cu) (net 7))
 (segment (start 187.325 104.14) (end 186.055 102.87) (width 0.25) (layer F.Cu) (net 8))
 (segment (start 187.325 106.68) (end 187.325 104.14) (width 0.25) (layer F.Cu) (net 8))
 (segment (start 186.055 107.95) (end 187.325 106.68) (width 0.25) (layer F.Cu) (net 8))
 (segment (start 186.055 109.22) (end 186.055 107.95) (width 0.25) (layer F.Cu) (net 8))
 (segment (start 186.055 102.87) (end 186.055 99.695) (width 0.25) (layer F.Cu) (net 8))
 (segment (start 188.595 109.22) (end 188.595 107.95) (width 0.25) (layer F.Cu) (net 9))
 (segment (start 188.595 107.95) (end 189.865 106.68) (width 0.25) (layer F.Cu) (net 9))
 (segment (start 189.865 106.68) (end 189.865 104.14) (width 0.25) (layer F.Cu) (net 9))
 (segment (start 189.865 104.14) (end 188.595 102.87) (width 0.25) (layer F.Cu) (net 9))
 (segment (start 188.595 100.946308) (end 189.855654 99.685654) (width 0.25) (layer F.Cu) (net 9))
 (segment (start 188.595 102.87) (end 188.595 100.946308) (width 0.25) (layer F.Cu) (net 9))
 (segment (start 191.135 109.22) (end 191.135 107.95) (width 0.25) (layer F.Cu) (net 10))
 (segment (start 191.135 107.95) (end 192.405 106.68) (width 0.25) (layer F.Cu) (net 10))
 (segment (start 192.405 106.68) (end 192.405 104.14) (width 0.25) (layer F.Cu) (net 10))
 (segment (start 192.405 104.14) (end 191.135 102.87) (width 0.25) (layer F.Cu) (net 10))
 (segment (start 193.675 109.22) (end 193.675 107.95) (width 0.25) (layer F.Cu) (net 4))
 (segment (start 193.675 107.95) (end 194.945 106.68) (width 0.25) (layer F.Cu) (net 4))
 (segment (start 194.945 106.68) (end 194.945 104.14) (width 0.25) (layer F.Cu) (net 4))
 (segment (start 194.945 104.14) (end 193.675 102.87) (width 0.25) (layer F.Cu) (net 4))
 (segment (start 193.675 102.87) (end 193.675 99.695) (width 0.25) (layer F.Cu) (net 4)))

